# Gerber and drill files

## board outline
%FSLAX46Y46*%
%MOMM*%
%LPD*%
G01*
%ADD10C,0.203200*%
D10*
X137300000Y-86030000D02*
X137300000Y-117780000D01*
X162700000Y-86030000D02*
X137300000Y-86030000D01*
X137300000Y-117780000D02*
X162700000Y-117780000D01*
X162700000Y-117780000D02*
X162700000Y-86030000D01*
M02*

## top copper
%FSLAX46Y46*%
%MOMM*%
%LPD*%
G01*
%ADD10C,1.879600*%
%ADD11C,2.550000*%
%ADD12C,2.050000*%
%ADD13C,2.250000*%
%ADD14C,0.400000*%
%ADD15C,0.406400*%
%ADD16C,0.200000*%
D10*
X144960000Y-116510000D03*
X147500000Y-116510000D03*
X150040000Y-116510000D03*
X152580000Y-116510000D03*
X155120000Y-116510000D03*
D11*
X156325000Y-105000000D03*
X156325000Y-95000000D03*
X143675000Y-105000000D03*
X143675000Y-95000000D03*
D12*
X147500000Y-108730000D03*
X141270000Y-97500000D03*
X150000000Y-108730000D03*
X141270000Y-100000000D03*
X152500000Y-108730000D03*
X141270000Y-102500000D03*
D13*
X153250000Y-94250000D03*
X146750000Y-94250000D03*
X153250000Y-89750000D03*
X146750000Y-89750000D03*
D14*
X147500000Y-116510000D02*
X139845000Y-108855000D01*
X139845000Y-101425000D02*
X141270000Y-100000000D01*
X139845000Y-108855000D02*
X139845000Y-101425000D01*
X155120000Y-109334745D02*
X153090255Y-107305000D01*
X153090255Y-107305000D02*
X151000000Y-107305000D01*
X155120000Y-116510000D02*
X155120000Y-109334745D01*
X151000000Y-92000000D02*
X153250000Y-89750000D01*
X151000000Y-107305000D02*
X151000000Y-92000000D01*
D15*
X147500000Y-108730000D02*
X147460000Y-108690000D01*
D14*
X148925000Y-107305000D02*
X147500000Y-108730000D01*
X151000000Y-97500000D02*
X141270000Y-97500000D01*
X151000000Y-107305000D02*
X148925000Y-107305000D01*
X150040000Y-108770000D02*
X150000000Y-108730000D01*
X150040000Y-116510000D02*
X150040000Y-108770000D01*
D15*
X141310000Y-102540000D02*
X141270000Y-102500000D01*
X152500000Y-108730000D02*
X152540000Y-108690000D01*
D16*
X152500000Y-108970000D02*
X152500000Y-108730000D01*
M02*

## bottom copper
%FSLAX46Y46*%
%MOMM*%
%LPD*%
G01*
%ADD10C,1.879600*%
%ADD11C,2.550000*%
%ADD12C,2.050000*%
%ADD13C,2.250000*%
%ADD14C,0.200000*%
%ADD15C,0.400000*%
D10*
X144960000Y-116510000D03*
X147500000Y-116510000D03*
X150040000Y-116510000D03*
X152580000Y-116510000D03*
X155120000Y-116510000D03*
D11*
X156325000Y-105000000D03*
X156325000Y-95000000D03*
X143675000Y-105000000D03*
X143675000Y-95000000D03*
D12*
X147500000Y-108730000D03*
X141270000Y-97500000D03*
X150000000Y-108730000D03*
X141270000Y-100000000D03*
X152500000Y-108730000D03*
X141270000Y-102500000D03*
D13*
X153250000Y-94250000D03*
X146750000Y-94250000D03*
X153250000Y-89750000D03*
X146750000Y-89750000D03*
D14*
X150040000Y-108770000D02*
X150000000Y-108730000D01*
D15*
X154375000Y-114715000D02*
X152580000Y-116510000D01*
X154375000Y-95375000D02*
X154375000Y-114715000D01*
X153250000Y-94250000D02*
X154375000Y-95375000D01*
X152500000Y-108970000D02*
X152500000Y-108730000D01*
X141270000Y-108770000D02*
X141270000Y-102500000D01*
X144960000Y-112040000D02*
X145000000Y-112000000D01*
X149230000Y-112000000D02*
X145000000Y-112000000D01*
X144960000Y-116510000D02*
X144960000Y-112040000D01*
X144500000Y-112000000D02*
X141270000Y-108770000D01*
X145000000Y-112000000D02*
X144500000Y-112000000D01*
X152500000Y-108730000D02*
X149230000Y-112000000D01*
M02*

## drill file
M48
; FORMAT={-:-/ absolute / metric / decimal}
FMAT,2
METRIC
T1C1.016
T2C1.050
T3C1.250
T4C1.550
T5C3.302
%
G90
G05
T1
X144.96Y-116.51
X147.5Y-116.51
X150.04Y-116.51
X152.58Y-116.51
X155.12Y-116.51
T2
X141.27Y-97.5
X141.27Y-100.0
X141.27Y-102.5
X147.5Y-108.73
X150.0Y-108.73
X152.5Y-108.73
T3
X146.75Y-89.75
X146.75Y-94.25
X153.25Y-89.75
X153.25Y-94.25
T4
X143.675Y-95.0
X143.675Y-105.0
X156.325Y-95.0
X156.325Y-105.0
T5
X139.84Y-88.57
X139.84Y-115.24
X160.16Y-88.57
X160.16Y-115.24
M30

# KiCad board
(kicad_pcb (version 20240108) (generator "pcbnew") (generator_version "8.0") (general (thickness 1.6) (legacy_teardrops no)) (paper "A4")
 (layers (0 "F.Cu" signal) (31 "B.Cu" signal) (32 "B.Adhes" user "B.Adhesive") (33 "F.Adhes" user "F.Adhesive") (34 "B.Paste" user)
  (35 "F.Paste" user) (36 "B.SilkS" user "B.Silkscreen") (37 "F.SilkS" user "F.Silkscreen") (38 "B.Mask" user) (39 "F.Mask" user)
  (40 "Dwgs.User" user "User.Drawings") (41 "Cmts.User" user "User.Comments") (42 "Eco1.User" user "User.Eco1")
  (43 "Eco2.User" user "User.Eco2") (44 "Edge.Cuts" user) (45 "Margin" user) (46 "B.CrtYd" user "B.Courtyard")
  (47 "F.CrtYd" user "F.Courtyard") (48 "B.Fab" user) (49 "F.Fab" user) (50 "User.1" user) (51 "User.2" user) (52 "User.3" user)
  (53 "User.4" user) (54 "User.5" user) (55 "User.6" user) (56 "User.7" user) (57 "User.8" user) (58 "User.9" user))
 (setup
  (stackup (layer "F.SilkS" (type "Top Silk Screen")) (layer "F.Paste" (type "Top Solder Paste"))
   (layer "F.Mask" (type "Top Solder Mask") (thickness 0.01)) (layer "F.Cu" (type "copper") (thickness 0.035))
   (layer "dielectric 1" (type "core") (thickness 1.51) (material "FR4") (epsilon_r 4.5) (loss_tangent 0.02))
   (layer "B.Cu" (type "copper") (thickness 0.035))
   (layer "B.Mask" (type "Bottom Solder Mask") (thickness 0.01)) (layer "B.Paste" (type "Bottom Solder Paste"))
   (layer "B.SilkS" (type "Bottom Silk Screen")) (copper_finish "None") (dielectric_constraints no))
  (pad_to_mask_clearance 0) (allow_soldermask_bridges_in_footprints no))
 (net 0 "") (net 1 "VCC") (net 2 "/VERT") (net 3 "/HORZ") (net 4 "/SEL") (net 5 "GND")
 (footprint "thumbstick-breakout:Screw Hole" (layer "F.Cu") (at 139.84 115.24)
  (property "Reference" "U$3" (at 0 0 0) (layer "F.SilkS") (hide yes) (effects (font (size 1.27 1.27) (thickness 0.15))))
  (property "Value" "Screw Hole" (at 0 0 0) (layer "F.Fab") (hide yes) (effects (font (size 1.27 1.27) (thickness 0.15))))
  (pad "" np_thru_hole circle (at 0 0) (size 3.302 3.302) (drill 3.302) (layers "F&B.Cu" "*.Mask")))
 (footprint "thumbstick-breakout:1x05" (layer "F.Cu") (at 150.04 116.51)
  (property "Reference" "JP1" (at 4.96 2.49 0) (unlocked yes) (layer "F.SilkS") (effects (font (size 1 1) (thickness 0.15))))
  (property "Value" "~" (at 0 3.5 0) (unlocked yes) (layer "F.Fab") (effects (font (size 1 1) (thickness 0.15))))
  (pad "1" thru_hole circle (at -5.08 0 270) (size 1.8796 1.8796) (drill 1.016) (layers "*.Cu" "*.Mask") (remove_unused_layers no)
   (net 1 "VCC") (solder_mask_margin 0.1) (thermal_bridge_angle 0))
  (pad "2" thru_hole circle (at -2.54 0 270) (size 1.8796 1.8796) (drill 1.016) (layers "*.Cu" "*.Mask") (remove_unused_layers no)
   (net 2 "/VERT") (solder_mask_margin 0.1) (thermal_bridge_angle 0))
  (pad "3" thru_hole circle (at 0 0 270) (size 1.8796 1.8796) (drill 1.016) (layers "*.Cu" "*.Mask") (remove_unused_layers no)
   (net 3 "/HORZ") (solder_mask_margin 0.1) (thermal_bridge_angle 0))
  (pad "4" thru_hole circle (at 2.54 0 270) (size 1.8796 1.8796) (drill 1.016) (layers "*.Cu" "*.Mask") (remove_unused_layers no)
   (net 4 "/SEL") (solder_mask_margin 0.1) (thermal_bridge_angle 0))
  (pad "5" thru_hole circle (at 5.08 0 270) (size 1.8796 1.8796) (drill 1.016) (layers "*.Cu" "*.Mask") (remove_unused_layers no)
   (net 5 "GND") (solder_mask_margin 0.1) (thermal_bridge_angle 0)))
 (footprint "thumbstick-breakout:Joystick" (layer "F.Cu") (at 150 100 180)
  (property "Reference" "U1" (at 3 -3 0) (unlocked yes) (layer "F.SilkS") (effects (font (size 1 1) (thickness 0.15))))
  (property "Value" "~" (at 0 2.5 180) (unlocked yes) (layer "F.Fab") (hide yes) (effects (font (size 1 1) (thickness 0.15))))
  (pad "" thru_hole circle (at -6.325 -5 180) (size 2.55 2.55) (drill 1.55) (layers "*.Cu" "*.Mask") (remove_unused_layers no)
   (solder_mask_margin 0.1))
  (pad "" thru_hole circle (at -6.325 5 180) (size 2.55 2.55) (drill 1.55) (layers "*.Cu" "*.Mask") (remove_unused_layers no)
   (solder_mask_margin 0.1))
  (pad "" thru_hole circle (at 6.325 -5 180) (size 2.55 2.55) (drill 1.55) (layers "*.Cu" "*.Mask") (remove_unused_layers no)
   (solder_mask_margin 0.1))
  (pad "" thru_hole circle (at 6.325 5 180) (size 2.55 2.55) (drill 1.55) (layers "*.Cu" "*.Mask") (remove_unused_layers no)
   (solder_mask_margin 0.1))
  (pad "1" thru_hole circle (at 2.5 -8.73 180) (size 2.05 2.05) (drill 1.05) (layers "*.Cu" "*.Mask") (remove_unused_layers no)
   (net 5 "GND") (solder_mask_margin 0.1))
  (pad "1'" thru_hole circle (at 8.73 2.5 180) (size 2.05 2.05) (drill 1.05) (layers "*.Cu" "*.Mask") (remove_unused_layers no)
   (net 5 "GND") (solder_mask_margin 0.1))
  (pad "2" thru_hole circle (at 0 -8.73 180) (size 2.05 2.05) (drill 1.05) (layers "*.Cu" "*.Mask") (remove_unused_layers no)
   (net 3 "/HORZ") (solder_mask_margin 0.1))
  (pad "2'" thru_hole circle (at 8.73 0 180) (size 2.05 2.05) (drill 1.05) (layers "*.Cu" "*.Mask") (remove_unused_layers no)
   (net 2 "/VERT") (solder_mask_margin 0.1))
  (pad "3" thru_hole circle (at -2.5 -8.73 180) (size 2.05 2.05) (drill 1.05) (layers "*.Cu" "*.Mask") (remove_unused_layers no)
   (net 1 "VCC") (solder_mask_margin 0.1))
  (pad "3'" thru_hole circle (at 8.73 -2.5 180) (size 2.05 2.05) (drill 1.05) (layers "*.Cu" "*.Mask") (remove_unused_layers no)
   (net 1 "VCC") (solder_mask_margin 0.1))
  (pad "a" thru_hole circle (at -3.25 5.75 180) (size 2.25 2.25) (drill 1.25) (layers "*.Cu" "*.Mask") (remove_unused_layers no)
   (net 4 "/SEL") (solder_mask_margin 0.1))
  (pad "b" thru_hole circle (at 3.25 5.75 180) (size 2.25 2.25) (drill 1.25) (layers "*.Cu" "*.Mask") (remove_unused_layers no)
   (solder_mask_margin 0.1))
  (pad "c" thru_hole circle (at -3.25 10.25 180) (size 2.25 2.25) (drill 1.25) (layers "*.Cu" "*.Mask") (remove_unused_layers no)
   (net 5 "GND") (solder_mask_margin 0.1))
  (pad "d" thru_hole circle (at 3.25 10.25 180) (size 2.25 2.25) (drill 1.25) (layers "*.Cu" "*.Mask") (remove_unused_layers no)
   (solder_mask_margin 0.1)))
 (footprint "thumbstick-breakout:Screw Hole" (layer "F.Cu") (at 160.16 115.24)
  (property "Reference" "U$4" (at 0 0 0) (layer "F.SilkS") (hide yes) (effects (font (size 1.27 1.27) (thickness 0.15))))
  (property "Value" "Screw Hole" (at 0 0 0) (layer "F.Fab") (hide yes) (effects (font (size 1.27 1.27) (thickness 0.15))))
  (pad "" np_thru_hole circle (at 0 0) (size 3.302 3.302) (drill 3.302) (layers "F&B.Cu" "*.Mask")))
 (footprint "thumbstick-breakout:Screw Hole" (layer "F.Cu") (at 160.16 88.57)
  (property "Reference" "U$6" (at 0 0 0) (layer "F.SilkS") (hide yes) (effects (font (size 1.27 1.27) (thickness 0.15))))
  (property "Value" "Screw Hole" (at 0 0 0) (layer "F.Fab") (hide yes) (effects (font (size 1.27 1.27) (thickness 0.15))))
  (pad "" np_thru_hole circle (at 0 0) (size 3.302 3.302) (drill 3.302) (layers "F&B.Cu" "*.Mask")))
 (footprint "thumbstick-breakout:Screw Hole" (layer "F.Cu") (at 139.84 88.57)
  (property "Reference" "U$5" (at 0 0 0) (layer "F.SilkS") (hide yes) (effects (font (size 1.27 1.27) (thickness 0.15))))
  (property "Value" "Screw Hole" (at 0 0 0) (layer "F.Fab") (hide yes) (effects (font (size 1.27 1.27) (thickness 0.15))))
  (pad "" np_thru_hole circle (at 0 0) (size 3.302 3.302) (drill 3.302) (layers "F&B.Cu" "*.Mask")))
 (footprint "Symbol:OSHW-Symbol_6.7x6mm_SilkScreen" (layer "B.Cu") (at 150 99.685893 180)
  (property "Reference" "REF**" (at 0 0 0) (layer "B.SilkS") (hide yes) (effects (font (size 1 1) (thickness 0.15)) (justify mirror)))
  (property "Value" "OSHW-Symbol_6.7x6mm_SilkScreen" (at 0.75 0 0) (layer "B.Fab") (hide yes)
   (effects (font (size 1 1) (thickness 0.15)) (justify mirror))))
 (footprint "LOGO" (layer "B.Cu") (at 157.5 87.5 180)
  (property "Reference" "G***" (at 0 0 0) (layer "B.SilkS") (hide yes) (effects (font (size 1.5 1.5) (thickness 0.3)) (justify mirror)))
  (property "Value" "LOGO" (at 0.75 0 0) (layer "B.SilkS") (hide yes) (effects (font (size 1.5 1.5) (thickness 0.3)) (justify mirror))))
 (gr_line (start 137.3 86.03) (end 137.3 117.78) (stroke (width 0.2032) (type solid)) (layer "Edge.Cuts"))
 (gr_line (start 162.7 86.03) (end 137.3 86.03) (stroke (width 0.2032) (type solid)) (layer "Edge.Cuts"))
 (gr_line (start 137.3 117.78) (end 162.7 117.78) (stroke (width 0.2032) (type solid)) (layer "Edge.Cuts"))
 (gr_line (start 162.7 117.78) (end 162.7 86.03) (stroke (width 0.2032) (type solid)) (layer "Edge.Cuts"))
 (segment (start 147.5 116.51) (end 139.845 108.855) (width 0.4) (layer "F.Cu") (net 2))
 (segment (start 139.845 101.425) (end 141.27 100) (width 0.4) (layer "F.Cu") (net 2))
 (segment (start 139.845 108.855) (end 139.845 101.425) (width 0.4) (layer "F.Cu") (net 2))
 (segment (start 155.12 109.334745) (end 153.090255 107.305) (width 0.4) (layer "F.Cu") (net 5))
 (segment (start 153.090255 107.305) (end 151 107.305) (width 0.4) (layer "F.Cu") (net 5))
 (segment (start 155.12 116.51) (end 155.12 109.334745) (width 0.4) (layer "F.Cu") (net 5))
 (segment (start 151 92) (end 153.25 89.75) (width 0.4) (layer "F.Cu") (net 5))
 (segment (start 151 107.305) (end 151 92) (width 0.4) (layer "F.Cu") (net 5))
 (segment (start 147.5 108.73) (end 147.46 108.69) (width 0.4064) (layer "F.Cu") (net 5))
 (segment (start 148.925 107.305) (end 147.5 108.73) (width 0.4) (layer "F.Cu") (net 5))
 (segment (start 151 97.5) (end 141.27 97.5) (width 0.4) (layer "F.Cu") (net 5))
 (segment (start 151 107.305) (end 148.925 107.305) (width 0.4) (layer "F.Cu") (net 5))
 (segment (start 150.04 108.77) (end 150 108.73) (width 0.4) (layer "F.Cu") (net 3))
 (segment (start 150.04 116.51) (end 150.04 108.77) (width 0.4) (layer "F.Cu") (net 3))
 (segment (start 150.04 108.77) (end 150 108.73) (width 0.2) (layer "B.Cu") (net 3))
 (segment (start 154.375 114.715) (end 152.58 116.51) (width 0.4) (layer "B.Cu") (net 4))
 (segment (start 154.375 95.375) (end 154.375 114.715) (width 0.4) (layer "B.Cu") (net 4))
 (segment (start 153.25 94.25) (end 154.375 95.375) (width 0.4) (layer "B.Cu") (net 4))
 (segment (start 141.31 102.54) (end 141.27 102.5) (width 0.4064) (layer "F.Cu") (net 1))
 (segment (start 152.5 108.73) (end 152.54 108.69) (width 0.4064) (layer "F.Cu") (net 1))
 (segment (start 152.5 108.97) (end 152.5 108.73) (width 0.2) (layer "F.Cu") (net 1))
 (segment (start 152.5 108.97) (end 152.5 108.73) (width 0.4) (layer "B.Cu") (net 1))
 (segment (start 141.27 108.77) (end 141.27 102.5) (width 0.4) (layer "B.Cu") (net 1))
 (segment (start 144.96 112.04) (end 145 112) (width 0.4) (layer "B.Cu") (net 1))
 (segment (start 149.23 112) (end 145 112) (width 0.4) (layer "B.Cu") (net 1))
 (segment (start 144.96 116.51) (end 144.96 112.04) (width 0.4) (layer "B.Cu") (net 1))
 (segment (start 144.5 112) (end 141.27 108.77) (width 0.4) (layer "B.Cu") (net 1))
 (segment (start 145 112) (end 144.5 112) (width 0.4) (layer "B.Cu") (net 1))
 (segment (start 152.5 108.73) (end 149.23 112) (width 0.4) (layer "B.Cu") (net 1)))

